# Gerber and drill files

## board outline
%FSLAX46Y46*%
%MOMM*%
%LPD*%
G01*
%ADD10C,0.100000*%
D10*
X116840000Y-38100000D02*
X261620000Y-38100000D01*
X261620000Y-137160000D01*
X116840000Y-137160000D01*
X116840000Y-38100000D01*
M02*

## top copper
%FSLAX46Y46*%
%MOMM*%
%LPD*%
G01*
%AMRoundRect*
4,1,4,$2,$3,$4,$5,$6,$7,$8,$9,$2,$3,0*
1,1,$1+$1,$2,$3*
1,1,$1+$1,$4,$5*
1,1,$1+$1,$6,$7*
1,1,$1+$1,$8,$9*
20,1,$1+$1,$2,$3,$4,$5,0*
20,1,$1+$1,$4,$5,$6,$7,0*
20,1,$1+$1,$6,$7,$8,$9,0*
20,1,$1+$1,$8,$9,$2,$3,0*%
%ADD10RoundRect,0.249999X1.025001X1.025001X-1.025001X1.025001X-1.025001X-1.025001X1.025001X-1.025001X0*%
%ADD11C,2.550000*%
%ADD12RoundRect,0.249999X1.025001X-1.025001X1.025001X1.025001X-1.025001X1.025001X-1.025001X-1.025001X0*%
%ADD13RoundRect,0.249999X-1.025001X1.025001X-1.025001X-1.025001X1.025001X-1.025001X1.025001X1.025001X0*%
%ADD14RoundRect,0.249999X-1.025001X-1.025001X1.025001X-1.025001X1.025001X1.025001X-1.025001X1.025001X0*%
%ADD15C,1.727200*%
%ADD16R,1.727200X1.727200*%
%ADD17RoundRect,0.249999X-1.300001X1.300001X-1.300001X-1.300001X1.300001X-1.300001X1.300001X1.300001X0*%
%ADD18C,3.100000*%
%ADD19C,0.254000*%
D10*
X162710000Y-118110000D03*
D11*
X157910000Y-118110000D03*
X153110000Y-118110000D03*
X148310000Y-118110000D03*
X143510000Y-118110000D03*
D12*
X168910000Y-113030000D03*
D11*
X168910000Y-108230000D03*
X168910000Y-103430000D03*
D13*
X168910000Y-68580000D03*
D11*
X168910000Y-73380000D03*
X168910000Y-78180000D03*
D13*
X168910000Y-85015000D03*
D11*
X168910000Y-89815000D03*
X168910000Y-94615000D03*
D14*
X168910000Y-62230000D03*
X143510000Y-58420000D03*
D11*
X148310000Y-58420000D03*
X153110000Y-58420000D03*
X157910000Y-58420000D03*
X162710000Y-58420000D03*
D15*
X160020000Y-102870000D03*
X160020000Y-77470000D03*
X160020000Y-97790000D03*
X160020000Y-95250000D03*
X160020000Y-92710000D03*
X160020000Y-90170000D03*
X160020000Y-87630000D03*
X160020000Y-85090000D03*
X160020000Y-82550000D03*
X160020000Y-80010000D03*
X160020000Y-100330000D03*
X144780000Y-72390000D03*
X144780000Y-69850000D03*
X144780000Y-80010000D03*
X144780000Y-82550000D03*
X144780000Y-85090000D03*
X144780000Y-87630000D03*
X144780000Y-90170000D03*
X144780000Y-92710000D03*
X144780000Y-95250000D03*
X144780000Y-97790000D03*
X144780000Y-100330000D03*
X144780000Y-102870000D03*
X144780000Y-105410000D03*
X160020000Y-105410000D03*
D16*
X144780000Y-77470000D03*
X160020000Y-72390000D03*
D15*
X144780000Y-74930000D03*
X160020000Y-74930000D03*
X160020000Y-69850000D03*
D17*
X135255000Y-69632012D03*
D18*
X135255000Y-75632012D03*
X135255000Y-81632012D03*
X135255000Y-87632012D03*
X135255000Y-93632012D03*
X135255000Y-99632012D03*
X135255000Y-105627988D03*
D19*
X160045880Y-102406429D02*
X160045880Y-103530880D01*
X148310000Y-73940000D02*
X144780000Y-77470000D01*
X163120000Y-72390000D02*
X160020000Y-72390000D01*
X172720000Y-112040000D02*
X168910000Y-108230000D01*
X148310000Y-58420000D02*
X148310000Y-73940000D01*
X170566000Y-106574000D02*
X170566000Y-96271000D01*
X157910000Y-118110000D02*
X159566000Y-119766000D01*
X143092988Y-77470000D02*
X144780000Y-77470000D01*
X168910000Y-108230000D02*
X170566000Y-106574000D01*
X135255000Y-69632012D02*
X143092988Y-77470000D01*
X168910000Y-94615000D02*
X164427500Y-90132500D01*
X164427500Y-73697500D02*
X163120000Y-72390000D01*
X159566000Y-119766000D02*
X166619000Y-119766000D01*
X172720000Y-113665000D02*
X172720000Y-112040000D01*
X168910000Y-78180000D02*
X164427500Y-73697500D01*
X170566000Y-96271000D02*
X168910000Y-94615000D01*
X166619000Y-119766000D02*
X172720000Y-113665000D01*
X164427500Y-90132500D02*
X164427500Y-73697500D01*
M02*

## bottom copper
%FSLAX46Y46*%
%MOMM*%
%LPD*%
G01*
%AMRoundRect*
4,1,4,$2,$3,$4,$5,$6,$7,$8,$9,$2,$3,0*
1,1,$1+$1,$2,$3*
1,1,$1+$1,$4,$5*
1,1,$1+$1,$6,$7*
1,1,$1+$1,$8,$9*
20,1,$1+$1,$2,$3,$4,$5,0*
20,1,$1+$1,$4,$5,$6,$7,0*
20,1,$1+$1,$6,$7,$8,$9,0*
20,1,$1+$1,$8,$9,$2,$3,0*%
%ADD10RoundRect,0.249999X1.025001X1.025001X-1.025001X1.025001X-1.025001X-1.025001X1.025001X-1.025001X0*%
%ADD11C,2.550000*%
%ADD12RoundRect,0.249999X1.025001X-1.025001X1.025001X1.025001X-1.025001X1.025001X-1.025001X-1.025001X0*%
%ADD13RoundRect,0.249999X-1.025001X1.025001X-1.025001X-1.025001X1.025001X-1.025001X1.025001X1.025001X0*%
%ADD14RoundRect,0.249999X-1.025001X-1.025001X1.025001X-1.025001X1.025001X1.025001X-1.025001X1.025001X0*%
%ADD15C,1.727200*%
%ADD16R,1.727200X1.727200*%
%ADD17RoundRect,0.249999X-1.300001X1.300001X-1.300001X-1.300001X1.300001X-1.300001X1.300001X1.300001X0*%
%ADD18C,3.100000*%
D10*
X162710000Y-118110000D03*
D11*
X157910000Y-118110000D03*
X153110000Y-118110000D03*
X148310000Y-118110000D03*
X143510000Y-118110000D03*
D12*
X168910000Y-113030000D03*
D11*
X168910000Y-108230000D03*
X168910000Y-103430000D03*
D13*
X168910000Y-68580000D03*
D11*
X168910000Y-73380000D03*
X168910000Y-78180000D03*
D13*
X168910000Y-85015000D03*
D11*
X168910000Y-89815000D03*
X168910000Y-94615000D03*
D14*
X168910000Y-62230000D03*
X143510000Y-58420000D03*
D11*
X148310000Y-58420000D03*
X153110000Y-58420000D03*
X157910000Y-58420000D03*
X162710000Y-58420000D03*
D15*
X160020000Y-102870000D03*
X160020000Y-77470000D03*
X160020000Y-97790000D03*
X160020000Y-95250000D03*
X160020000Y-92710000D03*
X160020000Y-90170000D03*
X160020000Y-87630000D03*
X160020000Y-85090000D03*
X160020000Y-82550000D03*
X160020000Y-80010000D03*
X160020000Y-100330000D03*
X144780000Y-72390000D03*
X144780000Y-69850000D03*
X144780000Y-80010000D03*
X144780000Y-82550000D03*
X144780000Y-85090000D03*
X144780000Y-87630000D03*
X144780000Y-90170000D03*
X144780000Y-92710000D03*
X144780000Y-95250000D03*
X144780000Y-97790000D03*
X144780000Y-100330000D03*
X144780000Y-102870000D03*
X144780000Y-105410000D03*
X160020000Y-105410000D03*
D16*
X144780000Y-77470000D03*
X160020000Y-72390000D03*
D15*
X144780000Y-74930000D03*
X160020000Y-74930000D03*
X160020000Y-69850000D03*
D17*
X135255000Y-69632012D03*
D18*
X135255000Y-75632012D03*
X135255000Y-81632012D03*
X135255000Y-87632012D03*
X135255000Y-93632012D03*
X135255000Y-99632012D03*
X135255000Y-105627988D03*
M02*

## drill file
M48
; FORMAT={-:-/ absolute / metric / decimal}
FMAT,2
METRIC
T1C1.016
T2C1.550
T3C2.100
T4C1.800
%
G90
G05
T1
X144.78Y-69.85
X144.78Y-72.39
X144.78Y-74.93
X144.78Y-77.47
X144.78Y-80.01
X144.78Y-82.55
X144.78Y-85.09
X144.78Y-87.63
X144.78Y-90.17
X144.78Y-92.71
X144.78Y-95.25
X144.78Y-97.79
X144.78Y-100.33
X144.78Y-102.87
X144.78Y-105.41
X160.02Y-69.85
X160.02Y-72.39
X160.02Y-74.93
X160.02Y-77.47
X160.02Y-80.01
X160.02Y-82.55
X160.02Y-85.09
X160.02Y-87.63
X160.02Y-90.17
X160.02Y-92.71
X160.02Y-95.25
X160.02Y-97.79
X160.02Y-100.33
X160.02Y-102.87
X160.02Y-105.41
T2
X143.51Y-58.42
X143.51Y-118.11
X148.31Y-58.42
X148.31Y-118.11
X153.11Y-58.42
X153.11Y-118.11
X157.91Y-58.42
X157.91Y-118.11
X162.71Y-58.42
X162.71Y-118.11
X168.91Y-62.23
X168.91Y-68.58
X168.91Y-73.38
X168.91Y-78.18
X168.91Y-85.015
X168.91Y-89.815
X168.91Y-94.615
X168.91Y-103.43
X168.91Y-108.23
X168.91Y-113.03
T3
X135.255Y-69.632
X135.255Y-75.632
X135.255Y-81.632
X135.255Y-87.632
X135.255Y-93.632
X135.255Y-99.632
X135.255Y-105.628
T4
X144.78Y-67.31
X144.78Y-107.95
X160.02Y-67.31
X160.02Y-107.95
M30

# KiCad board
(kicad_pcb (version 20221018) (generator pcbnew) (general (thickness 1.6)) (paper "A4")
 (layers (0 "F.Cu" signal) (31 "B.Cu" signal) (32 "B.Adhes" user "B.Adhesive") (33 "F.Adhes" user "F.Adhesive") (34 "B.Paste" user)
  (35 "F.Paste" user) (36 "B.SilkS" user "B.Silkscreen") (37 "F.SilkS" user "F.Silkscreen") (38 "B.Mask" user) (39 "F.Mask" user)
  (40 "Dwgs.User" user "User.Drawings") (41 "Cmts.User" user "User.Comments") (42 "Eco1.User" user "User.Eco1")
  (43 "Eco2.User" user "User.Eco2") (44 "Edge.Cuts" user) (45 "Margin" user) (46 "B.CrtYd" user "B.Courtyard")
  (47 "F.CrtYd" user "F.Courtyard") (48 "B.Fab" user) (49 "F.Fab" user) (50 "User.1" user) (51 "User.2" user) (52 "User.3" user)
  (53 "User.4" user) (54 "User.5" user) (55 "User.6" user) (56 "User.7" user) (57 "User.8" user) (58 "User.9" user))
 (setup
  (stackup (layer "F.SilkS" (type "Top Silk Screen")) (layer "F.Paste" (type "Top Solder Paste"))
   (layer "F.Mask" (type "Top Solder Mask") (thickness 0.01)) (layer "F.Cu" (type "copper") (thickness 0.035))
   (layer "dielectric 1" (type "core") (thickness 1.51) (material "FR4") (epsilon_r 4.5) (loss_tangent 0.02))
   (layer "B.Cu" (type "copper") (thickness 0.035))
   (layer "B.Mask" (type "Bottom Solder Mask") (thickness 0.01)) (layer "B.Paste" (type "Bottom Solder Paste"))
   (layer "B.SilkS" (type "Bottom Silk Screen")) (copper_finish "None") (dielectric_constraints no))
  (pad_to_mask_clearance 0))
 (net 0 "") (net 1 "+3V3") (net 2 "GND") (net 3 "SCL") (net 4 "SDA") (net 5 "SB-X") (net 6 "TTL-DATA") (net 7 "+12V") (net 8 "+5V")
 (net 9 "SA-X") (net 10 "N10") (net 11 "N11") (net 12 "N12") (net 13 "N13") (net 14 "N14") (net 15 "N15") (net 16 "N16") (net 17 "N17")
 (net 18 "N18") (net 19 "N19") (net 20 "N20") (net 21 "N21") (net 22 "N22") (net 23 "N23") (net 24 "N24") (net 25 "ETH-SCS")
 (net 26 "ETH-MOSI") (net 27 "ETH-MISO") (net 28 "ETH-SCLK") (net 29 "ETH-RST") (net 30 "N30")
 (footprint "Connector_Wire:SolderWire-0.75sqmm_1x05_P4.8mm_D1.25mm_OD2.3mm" (layer "F.Cu") (at 162.71 118.11 180)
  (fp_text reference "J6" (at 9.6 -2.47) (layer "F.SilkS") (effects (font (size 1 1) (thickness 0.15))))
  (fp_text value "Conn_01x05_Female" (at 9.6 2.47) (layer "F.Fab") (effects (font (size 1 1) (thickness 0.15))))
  (pad "1" thru_hole roundrect (at 0 0 180) (size 2.55 2.55) (drill 1.55) (layers "*.Cu" "*.Mask") (roundrect_rratio 0.098039)
   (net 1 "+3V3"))
  (pad "2" thru_hole circle (at 4.8 0 180) (size 2.55 2.55) (drill 1.55) (layers "*.Cu" "*.Mask") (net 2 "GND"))
  (pad "3" thru_hole circle (at 9.6 0 180) (size 2.55 2.55) (drill 1.55) (layers "*.Cu" "*.Mask") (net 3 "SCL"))
  (pad "4" thru_hole circle (at 14.4 0 180) (size 2.55 2.55) (drill 1.55) (layers "*.Cu" "*.Mask") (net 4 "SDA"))
  (pad "5" thru_hole circle (at 19.2 0 180) (size 2.55 2.55) (drill 1.55) (layers "*.Cu" "*.Mask") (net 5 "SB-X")))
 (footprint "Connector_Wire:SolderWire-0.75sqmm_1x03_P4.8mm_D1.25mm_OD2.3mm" (layer "F.Cu") (at 168.91 113.03 90)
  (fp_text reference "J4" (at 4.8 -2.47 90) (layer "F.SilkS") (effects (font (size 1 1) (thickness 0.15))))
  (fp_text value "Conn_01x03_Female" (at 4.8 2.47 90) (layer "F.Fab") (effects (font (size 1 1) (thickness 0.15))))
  (pad "1" thru_hole roundrect (at 0 0 90) (size 2.55 2.55) (drill 1.55) (layers "*.Cu" "*.Mask") (roundrect_rratio 0.098039) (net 1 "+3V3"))
  (pad "2" thru_hole circle (at 4.8 0 90) (size 2.55 2.55) (drill 1.55) (layers "*.Cu" "*.Mask") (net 2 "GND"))
  (pad "3" thru_hole circle (at 9.6 0 90) (size 2.55 2.55) (drill 1.55) (layers "*.Cu" "*.Mask") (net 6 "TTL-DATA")))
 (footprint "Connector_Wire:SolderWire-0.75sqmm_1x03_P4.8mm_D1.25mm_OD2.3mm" (layer "F.Cu") (at 168.91 68.58 -90)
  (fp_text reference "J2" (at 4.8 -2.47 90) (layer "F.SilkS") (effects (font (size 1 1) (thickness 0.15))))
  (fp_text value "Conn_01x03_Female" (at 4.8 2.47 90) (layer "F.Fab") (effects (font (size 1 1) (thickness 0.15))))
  (pad "1" thru_hole roundrect (at 0 0 270) (size 2.55 2.55) (drill 1.55) (layers "*.Cu" "*.Mask") (roundrect_rratio 0.098039)
   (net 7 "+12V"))
  (pad "2" thru_hole circle (at 4.8 0 270) (size 2.55 2.55) (drill 1.55) (layers "*.Cu" "*.Mask") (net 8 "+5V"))
  (pad "3" thru_hole circle (at 9.6 0 270) (size 2.55 2.55) (drill 1.55) (layers "*.Cu" "*.Mask") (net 2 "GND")))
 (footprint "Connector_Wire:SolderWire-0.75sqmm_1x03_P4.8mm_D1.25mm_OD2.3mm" (layer "F.Cu") (at 168.91 85.015 -90)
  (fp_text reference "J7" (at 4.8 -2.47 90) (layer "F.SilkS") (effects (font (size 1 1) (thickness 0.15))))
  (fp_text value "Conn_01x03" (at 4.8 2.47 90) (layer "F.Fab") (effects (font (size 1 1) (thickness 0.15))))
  (pad "1" thru_hole roundrect (at 0 0 270) (size 2.55 2.55) (drill 1.55) (layers "*.Cu" "*.Mask") (roundrect_rratio 0.098039)
   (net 7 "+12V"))
  (pad "2" thru_hole circle (at 4.8 0 270) (size 2.55 2.55) (drill 1.55) (layers "*.Cu" "*.Mask") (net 8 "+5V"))
  (pad "3" thru_hole circle (at 9.6 0 270) (size 2.55 2.55) (drill 1.55) (layers "*.Cu" "*.Mask") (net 2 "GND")))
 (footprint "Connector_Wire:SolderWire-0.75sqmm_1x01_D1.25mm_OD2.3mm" (layer "F.Cu") (at 168.91 62.23)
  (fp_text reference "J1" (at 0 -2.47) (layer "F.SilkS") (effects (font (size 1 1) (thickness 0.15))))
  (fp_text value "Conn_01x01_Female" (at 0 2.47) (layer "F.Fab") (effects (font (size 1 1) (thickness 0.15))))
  (pad "1" thru_hole roundrect (at 0 0) (size 2.55 2.55) (drill 1.55) (layers "*.Cu" "*.Mask") (roundrect_rratio 0.098039) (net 7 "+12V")))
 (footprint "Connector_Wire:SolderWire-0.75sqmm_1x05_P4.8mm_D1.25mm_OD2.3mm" (layer "F.Cu") (at 143.51 58.42)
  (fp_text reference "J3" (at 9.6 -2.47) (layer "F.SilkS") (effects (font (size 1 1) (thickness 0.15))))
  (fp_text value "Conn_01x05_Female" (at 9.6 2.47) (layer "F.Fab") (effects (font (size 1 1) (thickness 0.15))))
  (pad "1" thru_hole roundrect (at 0 0) (size 2.55 2.55) (drill 1.55) (layers "*.Cu" "*.Mask") (roundrect_rratio 0.098039) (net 1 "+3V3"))
  (pad "2" thru_hole circle (at 4.8 0) (size 2.55 2.55) (drill 1.55) (layers "*.Cu" "*.Mask") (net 2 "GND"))
  (pad "3" thru_hole circle (at 9.6 0) (size 2.55 2.55) (drill 1.55) (layers "*.Cu" "*.Mask") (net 4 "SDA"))
  (pad "4" thru_hole circle (at 14.4 0) (size 2.55 2.55) (drill 1.55) (layers "*.Cu" "*.Mask") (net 3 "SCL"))
  (pad "5" thru_hole circle (at 19.2 0) (size 2.55 2.55) (drill 1.55) (layers "*.Cu" "*.Mask") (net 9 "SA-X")))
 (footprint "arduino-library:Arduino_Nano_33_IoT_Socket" (layer "F.Cu") (at 152.4 109.22)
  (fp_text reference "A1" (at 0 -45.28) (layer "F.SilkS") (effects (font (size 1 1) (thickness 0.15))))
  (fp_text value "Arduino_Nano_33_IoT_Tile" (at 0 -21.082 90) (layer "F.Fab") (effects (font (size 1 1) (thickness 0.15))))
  (pad "" np_thru_hole circle (at -7.62 -41.91) (size 1.8 1.8) (drill 1.8) (layers "F&B.Cu" "*.Mask"))
  (pad "" np_thru_hole circle (at -7.62 -1.27) (size 1.8 1.8) (drill 1.8) (layers "F&B.Cu" "*.Mask"))
  (pad "" np_thru_hole circle (at 7.62 -41.91) (size 1.8 1.8) (drill 1.8) (layers "F&B.Cu" "*.Mask"))
  (pad "" np_thru_hole circle (at 7.62 -1.27) (size 1.8 1.8) (drill 1.8) (layers "F&B.Cu" "*.Mask"))
  (pad "3V3" thru_hole circle (at 7.62 -6.35) (size 1.7272 1.7272) (drill 1.016) (layers "*.Cu" "*.Mask") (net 1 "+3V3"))
  (pad "5V" thru_hole circle (at 7.62 -31.75) (size 1.7272 1.7272) (drill 1.016) (layers "*.Cu" "*.Mask") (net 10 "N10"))
  (pad "A0" thru_hole circle (at 7.62 -11.43) (size 1.7272 1.7272) (drill 1.016) (layers "*.Cu" "*.Mask") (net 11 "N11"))
  (pad "A1" thru_hole circle (at 7.62 -13.97) (size 1.7272 1.7272) (drill 1.016) (layers "*.Cu" "*.Mask") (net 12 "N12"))
  (pad "A2" thru_hole circle (at 7.62 -16.51) (size 1.7272 1.7272) (drill 1.016) (layers "*.Cu" "*.Mask") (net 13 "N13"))
  (pad "A3" thru_hole circle (at 7.62 -19.05) (size 1.7272 1.7272) (drill 1.016) (layers "*.Cu" "*.Mask") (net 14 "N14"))
  (pad "A4" thru_hole circle (at 7.62 -21.59) (size 1.7272 1.7272) (drill 1.016) (layers "*.Cu" "*.Mask") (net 4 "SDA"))
  (pad "A5" thru_hole circle (at 7.62 -24.13) (size 1.7272 1.7272) (drill 1.016) (layers "*.Cu" "*.Mask") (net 3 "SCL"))
  (pad "A6" thru_hole circle (at 7.62 -26.67) (size 1.7272 1.7272) (drill 1.016) (layers "*.Cu" "*.Mask") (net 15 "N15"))
  (pad "A7" thru_hole circle (at 7.62 -29.21) (size 1.7272 1.7272) (drill 1.016) (layers "*.Cu" "*.Mask") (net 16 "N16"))
  (pad "AREF" thru_hole circle (at 7.62 -8.89) (size 1.7272 1.7272) (drill 1.016) (layers "*.Cu" "*.Mask") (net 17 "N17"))
  (pad "D0" thru_hole circle (at -7.62 -36.83) (size 1.7272 1.7272) (drill 1.016) (layers "*.Cu" "*.Mask") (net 6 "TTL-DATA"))
  (pad "D1" thru_hole circle (at -7.62 -39.37) (size 1.7272 1.7272) (drill 1.016) (layers "*.Cu" "*.Mask") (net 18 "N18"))
  (pad "D2" thru_hole circle (at -7.62 -29.21) (size 1.7272 1.7272) (drill 1.016) (layers "*.Cu" "*.Mask") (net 9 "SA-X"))
  (pad "D3" thru_hole circle (at -7.62 -26.67) (size 1.7272 1.7272) (drill 1.016) (layers "*.Cu" "*.Mask") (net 5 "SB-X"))
  (pad "D4" thru_hole circle (at -7.62 -24.13) (size 1.7272 1.7272) (drill 1.016) (layers "*.Cu" "*.Mask") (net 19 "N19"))
  (pad "D5" thru_hole circle (at -7.62 -21.59) (size 1.7272 1.7272) (drill 1.016) (layers "*.Cu" "*.Mask") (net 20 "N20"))
  (pad "D6" thru_hole circle (at -7.62 -19.05) (size 1.7272 1.7272) (drill 1.016) (layers "*.Cu" "*.Mask") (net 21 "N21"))
  (pad "D7" thru_hole circle (at -7.62 -16.51) (size 1.7272 1.7272) (drill 1.016) (layers "*.Cu" "*.Mask") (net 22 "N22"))
  (pad "D8" thru_hole circle (at -7.62 -13.97) (size 1.7272 1.7272) (drill 1.016) (layers "*.Cu" "*.Mask") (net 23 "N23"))
  (pad "D9" thru_hole circle (at -7.62 -11.43) (size 1.7272 1.7272) (drill 1.016) (layers "*.Cu" "*.Mask") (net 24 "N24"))
  (pad "D10" thru_hole circle (at -7.62 -8.89) (size 1.7272 1.7272) (drill 1.016) (layers "*.Cu" "*.Mask") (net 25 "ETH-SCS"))
  (pad "D11" thru_hole circle (at -7.62 -6.35) (size 1.7272 1.7272) (drill 1.016) (layers "*.Cu" "*.Mask") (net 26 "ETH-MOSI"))
  (pad "D12" thru_hole circle (at -7.62 -3.81) (size 1.7272 1.7272) (drill 1.016) (layers "*.Cu" "*.Mask") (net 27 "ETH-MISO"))
  (pad "D13" thru_hole circle (at 7.62 -3.81) (size 1.7272 1.7272) (drill 1.016) (layers "*.Cu" "*.Mask") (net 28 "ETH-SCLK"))
  (pad "GND1" thru_hole rect (at -7.62 -31.75) (size 1.7272 1.7272) (drill 1.016) (layers "*.Cu" "*.Mask") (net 2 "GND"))
  (pad "GND2" thru_hole rect (at 7.62 -36.83) (size 1.7272 1.7272) (drill 1.016) (layers "*.Cu" "*.Mask") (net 2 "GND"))
  (pad "RST1" thru_hole circle (at -7.62 -34.29) (size 1.7272 1.7272) (drill 1.016) (layers "*.Cu" "*.Mask") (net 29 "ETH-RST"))
  (pad "RST2" thru_hole circle (at 7.62 -34.29) (size 1.7272 1.7272) (drill 1.016) (layers "*.Cu" "*.Mask") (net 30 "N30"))
  (pad "VIN" thru_hole circle (at 7.62 -39.37) (size 1.7272 1.7272) (drill 1.016) (layers "*.Cu" "*.Mask") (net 8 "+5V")))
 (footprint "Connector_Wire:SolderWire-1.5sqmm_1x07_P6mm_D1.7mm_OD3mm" (layer "F.Cu") (at 135.255 69.632012 -90)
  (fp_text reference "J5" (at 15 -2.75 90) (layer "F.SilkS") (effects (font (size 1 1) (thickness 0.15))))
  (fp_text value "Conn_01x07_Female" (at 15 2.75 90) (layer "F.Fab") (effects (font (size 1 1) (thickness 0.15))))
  (pad "1" thru_hole roundrect (at 0 0 270) (size 3.1 3.1) (drill 2.1) (layers "*.Cu" "*.Mask") (roundrect_rratio 0.080645) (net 2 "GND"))
  (pad "2" thru_hole circle (at 6 0 270) (size 3.1 3.1) (drill 2.1) (layers "*.Cu" "*.Mask") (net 28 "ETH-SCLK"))
  (pad "3" thru_hole circle (at 12 0 270) (size 3.1 3.1) (drill 2.1) (layers "*.Cu" "*.Mask") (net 25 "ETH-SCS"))
  (pad "4" thru_hole circle (at 18 0 270) (size 3.1 3.1) (drill 2.1) (layers "*.Cu" "*.Mask") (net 26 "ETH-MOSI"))
  (pad "5" thru_hole circle (at 24 0 270) (size 3.1 3.1) (drill 2.1) (layers "*.Cu" "*.Mask") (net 27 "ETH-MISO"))
  (pad "6" thru_hole circle (at 30 0 270) (size 3.1 3.1) (drill 2.1) (layers "*.Cu" "*.Mask") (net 1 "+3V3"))
  (pad "7" thru_hole circle (at 35.995976 0 270) (size 3.1 3.1) (drill 2.1) (layers "*.Cu" "*.Mask") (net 29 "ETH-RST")))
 (gr_rect (start 116.84 38.1) (end 261.62 137.16) (stroke (width 0.1) (type solid)) (fill none) (layer "Edge.Cuts"))
 (segment (start 160.04588 102.406429) (end 160.04588 103.53088) (width 0.254) (layer "F.Cu") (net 1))
 (segment (start 148.31 73.94) (end 144.78 77.47) (width 0.254) (layer "F.Cu") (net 2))
 (segment (start 163.12 72.39) (end 160.02 72.39) (width 0.254) (layer "F.Cu") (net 2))
 (segment (start 172.72 112.04) (end 168.91 108.23) (width 0.254) (layer "F.Cu") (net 2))
 (segment (start 148.31 58.42) (end 148.31 73.94) (width 0.254) (layer "F.Cu") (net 2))
 (segment (start 170.566 106.574) (end 170.566 96.271) (width 0.254) (layer "F.Cu") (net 2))
 (segment (start 157.91 118.11) (end 159.566 119.766) (width 0.254) (layer "F.Cu") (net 2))
 (segment (start 143.092988 77.47) (end 144.78 77.47) (width 0.254) (layer "F.Cu") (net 2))
 (segment (start 168.91 108.23) (end 170.566 106.574) (width 0.254) (layer "F.Cu") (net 2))
 (segment (start 135.255 69.632012) (end 143.092988 77.47) (width 0.254) (layer "F.Cu") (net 2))
 (segment (start 168.91 94.615) (end 164.4275 90.1325) (width 0.254) (layer "F.Cu") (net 2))
 (segment (start 164.4275 73.6975) (end 163.12 72.39) (width 0.254) (layer "F.Cu") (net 2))
 (segment (start 159.566 119.766) (end 166.619 119.766) (width 0.254) (layer "F.Cu") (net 2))
 (segment (start 172.72 113.665) (end 172.72 112.04) (width 0.254) (layer "F.Cu") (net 2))
 (segment (start 168.91 78.18) (end 164.4275 73.6975) (width 0.254) (layer "F.Cu") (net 2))
 (segment (start 170.566 96.271) (end 168.91 94.615) (width 0.254) (layer "F.Cu") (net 2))
 (segment (start 166.619 119.766) (end 172.72 113.665) (width 0.254) (layer "F.Cu") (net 2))
 (segment (start 164.4275 90.1325) (end 164.4275 73.6975) (width 0.254) (layer "F.Cu") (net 2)))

